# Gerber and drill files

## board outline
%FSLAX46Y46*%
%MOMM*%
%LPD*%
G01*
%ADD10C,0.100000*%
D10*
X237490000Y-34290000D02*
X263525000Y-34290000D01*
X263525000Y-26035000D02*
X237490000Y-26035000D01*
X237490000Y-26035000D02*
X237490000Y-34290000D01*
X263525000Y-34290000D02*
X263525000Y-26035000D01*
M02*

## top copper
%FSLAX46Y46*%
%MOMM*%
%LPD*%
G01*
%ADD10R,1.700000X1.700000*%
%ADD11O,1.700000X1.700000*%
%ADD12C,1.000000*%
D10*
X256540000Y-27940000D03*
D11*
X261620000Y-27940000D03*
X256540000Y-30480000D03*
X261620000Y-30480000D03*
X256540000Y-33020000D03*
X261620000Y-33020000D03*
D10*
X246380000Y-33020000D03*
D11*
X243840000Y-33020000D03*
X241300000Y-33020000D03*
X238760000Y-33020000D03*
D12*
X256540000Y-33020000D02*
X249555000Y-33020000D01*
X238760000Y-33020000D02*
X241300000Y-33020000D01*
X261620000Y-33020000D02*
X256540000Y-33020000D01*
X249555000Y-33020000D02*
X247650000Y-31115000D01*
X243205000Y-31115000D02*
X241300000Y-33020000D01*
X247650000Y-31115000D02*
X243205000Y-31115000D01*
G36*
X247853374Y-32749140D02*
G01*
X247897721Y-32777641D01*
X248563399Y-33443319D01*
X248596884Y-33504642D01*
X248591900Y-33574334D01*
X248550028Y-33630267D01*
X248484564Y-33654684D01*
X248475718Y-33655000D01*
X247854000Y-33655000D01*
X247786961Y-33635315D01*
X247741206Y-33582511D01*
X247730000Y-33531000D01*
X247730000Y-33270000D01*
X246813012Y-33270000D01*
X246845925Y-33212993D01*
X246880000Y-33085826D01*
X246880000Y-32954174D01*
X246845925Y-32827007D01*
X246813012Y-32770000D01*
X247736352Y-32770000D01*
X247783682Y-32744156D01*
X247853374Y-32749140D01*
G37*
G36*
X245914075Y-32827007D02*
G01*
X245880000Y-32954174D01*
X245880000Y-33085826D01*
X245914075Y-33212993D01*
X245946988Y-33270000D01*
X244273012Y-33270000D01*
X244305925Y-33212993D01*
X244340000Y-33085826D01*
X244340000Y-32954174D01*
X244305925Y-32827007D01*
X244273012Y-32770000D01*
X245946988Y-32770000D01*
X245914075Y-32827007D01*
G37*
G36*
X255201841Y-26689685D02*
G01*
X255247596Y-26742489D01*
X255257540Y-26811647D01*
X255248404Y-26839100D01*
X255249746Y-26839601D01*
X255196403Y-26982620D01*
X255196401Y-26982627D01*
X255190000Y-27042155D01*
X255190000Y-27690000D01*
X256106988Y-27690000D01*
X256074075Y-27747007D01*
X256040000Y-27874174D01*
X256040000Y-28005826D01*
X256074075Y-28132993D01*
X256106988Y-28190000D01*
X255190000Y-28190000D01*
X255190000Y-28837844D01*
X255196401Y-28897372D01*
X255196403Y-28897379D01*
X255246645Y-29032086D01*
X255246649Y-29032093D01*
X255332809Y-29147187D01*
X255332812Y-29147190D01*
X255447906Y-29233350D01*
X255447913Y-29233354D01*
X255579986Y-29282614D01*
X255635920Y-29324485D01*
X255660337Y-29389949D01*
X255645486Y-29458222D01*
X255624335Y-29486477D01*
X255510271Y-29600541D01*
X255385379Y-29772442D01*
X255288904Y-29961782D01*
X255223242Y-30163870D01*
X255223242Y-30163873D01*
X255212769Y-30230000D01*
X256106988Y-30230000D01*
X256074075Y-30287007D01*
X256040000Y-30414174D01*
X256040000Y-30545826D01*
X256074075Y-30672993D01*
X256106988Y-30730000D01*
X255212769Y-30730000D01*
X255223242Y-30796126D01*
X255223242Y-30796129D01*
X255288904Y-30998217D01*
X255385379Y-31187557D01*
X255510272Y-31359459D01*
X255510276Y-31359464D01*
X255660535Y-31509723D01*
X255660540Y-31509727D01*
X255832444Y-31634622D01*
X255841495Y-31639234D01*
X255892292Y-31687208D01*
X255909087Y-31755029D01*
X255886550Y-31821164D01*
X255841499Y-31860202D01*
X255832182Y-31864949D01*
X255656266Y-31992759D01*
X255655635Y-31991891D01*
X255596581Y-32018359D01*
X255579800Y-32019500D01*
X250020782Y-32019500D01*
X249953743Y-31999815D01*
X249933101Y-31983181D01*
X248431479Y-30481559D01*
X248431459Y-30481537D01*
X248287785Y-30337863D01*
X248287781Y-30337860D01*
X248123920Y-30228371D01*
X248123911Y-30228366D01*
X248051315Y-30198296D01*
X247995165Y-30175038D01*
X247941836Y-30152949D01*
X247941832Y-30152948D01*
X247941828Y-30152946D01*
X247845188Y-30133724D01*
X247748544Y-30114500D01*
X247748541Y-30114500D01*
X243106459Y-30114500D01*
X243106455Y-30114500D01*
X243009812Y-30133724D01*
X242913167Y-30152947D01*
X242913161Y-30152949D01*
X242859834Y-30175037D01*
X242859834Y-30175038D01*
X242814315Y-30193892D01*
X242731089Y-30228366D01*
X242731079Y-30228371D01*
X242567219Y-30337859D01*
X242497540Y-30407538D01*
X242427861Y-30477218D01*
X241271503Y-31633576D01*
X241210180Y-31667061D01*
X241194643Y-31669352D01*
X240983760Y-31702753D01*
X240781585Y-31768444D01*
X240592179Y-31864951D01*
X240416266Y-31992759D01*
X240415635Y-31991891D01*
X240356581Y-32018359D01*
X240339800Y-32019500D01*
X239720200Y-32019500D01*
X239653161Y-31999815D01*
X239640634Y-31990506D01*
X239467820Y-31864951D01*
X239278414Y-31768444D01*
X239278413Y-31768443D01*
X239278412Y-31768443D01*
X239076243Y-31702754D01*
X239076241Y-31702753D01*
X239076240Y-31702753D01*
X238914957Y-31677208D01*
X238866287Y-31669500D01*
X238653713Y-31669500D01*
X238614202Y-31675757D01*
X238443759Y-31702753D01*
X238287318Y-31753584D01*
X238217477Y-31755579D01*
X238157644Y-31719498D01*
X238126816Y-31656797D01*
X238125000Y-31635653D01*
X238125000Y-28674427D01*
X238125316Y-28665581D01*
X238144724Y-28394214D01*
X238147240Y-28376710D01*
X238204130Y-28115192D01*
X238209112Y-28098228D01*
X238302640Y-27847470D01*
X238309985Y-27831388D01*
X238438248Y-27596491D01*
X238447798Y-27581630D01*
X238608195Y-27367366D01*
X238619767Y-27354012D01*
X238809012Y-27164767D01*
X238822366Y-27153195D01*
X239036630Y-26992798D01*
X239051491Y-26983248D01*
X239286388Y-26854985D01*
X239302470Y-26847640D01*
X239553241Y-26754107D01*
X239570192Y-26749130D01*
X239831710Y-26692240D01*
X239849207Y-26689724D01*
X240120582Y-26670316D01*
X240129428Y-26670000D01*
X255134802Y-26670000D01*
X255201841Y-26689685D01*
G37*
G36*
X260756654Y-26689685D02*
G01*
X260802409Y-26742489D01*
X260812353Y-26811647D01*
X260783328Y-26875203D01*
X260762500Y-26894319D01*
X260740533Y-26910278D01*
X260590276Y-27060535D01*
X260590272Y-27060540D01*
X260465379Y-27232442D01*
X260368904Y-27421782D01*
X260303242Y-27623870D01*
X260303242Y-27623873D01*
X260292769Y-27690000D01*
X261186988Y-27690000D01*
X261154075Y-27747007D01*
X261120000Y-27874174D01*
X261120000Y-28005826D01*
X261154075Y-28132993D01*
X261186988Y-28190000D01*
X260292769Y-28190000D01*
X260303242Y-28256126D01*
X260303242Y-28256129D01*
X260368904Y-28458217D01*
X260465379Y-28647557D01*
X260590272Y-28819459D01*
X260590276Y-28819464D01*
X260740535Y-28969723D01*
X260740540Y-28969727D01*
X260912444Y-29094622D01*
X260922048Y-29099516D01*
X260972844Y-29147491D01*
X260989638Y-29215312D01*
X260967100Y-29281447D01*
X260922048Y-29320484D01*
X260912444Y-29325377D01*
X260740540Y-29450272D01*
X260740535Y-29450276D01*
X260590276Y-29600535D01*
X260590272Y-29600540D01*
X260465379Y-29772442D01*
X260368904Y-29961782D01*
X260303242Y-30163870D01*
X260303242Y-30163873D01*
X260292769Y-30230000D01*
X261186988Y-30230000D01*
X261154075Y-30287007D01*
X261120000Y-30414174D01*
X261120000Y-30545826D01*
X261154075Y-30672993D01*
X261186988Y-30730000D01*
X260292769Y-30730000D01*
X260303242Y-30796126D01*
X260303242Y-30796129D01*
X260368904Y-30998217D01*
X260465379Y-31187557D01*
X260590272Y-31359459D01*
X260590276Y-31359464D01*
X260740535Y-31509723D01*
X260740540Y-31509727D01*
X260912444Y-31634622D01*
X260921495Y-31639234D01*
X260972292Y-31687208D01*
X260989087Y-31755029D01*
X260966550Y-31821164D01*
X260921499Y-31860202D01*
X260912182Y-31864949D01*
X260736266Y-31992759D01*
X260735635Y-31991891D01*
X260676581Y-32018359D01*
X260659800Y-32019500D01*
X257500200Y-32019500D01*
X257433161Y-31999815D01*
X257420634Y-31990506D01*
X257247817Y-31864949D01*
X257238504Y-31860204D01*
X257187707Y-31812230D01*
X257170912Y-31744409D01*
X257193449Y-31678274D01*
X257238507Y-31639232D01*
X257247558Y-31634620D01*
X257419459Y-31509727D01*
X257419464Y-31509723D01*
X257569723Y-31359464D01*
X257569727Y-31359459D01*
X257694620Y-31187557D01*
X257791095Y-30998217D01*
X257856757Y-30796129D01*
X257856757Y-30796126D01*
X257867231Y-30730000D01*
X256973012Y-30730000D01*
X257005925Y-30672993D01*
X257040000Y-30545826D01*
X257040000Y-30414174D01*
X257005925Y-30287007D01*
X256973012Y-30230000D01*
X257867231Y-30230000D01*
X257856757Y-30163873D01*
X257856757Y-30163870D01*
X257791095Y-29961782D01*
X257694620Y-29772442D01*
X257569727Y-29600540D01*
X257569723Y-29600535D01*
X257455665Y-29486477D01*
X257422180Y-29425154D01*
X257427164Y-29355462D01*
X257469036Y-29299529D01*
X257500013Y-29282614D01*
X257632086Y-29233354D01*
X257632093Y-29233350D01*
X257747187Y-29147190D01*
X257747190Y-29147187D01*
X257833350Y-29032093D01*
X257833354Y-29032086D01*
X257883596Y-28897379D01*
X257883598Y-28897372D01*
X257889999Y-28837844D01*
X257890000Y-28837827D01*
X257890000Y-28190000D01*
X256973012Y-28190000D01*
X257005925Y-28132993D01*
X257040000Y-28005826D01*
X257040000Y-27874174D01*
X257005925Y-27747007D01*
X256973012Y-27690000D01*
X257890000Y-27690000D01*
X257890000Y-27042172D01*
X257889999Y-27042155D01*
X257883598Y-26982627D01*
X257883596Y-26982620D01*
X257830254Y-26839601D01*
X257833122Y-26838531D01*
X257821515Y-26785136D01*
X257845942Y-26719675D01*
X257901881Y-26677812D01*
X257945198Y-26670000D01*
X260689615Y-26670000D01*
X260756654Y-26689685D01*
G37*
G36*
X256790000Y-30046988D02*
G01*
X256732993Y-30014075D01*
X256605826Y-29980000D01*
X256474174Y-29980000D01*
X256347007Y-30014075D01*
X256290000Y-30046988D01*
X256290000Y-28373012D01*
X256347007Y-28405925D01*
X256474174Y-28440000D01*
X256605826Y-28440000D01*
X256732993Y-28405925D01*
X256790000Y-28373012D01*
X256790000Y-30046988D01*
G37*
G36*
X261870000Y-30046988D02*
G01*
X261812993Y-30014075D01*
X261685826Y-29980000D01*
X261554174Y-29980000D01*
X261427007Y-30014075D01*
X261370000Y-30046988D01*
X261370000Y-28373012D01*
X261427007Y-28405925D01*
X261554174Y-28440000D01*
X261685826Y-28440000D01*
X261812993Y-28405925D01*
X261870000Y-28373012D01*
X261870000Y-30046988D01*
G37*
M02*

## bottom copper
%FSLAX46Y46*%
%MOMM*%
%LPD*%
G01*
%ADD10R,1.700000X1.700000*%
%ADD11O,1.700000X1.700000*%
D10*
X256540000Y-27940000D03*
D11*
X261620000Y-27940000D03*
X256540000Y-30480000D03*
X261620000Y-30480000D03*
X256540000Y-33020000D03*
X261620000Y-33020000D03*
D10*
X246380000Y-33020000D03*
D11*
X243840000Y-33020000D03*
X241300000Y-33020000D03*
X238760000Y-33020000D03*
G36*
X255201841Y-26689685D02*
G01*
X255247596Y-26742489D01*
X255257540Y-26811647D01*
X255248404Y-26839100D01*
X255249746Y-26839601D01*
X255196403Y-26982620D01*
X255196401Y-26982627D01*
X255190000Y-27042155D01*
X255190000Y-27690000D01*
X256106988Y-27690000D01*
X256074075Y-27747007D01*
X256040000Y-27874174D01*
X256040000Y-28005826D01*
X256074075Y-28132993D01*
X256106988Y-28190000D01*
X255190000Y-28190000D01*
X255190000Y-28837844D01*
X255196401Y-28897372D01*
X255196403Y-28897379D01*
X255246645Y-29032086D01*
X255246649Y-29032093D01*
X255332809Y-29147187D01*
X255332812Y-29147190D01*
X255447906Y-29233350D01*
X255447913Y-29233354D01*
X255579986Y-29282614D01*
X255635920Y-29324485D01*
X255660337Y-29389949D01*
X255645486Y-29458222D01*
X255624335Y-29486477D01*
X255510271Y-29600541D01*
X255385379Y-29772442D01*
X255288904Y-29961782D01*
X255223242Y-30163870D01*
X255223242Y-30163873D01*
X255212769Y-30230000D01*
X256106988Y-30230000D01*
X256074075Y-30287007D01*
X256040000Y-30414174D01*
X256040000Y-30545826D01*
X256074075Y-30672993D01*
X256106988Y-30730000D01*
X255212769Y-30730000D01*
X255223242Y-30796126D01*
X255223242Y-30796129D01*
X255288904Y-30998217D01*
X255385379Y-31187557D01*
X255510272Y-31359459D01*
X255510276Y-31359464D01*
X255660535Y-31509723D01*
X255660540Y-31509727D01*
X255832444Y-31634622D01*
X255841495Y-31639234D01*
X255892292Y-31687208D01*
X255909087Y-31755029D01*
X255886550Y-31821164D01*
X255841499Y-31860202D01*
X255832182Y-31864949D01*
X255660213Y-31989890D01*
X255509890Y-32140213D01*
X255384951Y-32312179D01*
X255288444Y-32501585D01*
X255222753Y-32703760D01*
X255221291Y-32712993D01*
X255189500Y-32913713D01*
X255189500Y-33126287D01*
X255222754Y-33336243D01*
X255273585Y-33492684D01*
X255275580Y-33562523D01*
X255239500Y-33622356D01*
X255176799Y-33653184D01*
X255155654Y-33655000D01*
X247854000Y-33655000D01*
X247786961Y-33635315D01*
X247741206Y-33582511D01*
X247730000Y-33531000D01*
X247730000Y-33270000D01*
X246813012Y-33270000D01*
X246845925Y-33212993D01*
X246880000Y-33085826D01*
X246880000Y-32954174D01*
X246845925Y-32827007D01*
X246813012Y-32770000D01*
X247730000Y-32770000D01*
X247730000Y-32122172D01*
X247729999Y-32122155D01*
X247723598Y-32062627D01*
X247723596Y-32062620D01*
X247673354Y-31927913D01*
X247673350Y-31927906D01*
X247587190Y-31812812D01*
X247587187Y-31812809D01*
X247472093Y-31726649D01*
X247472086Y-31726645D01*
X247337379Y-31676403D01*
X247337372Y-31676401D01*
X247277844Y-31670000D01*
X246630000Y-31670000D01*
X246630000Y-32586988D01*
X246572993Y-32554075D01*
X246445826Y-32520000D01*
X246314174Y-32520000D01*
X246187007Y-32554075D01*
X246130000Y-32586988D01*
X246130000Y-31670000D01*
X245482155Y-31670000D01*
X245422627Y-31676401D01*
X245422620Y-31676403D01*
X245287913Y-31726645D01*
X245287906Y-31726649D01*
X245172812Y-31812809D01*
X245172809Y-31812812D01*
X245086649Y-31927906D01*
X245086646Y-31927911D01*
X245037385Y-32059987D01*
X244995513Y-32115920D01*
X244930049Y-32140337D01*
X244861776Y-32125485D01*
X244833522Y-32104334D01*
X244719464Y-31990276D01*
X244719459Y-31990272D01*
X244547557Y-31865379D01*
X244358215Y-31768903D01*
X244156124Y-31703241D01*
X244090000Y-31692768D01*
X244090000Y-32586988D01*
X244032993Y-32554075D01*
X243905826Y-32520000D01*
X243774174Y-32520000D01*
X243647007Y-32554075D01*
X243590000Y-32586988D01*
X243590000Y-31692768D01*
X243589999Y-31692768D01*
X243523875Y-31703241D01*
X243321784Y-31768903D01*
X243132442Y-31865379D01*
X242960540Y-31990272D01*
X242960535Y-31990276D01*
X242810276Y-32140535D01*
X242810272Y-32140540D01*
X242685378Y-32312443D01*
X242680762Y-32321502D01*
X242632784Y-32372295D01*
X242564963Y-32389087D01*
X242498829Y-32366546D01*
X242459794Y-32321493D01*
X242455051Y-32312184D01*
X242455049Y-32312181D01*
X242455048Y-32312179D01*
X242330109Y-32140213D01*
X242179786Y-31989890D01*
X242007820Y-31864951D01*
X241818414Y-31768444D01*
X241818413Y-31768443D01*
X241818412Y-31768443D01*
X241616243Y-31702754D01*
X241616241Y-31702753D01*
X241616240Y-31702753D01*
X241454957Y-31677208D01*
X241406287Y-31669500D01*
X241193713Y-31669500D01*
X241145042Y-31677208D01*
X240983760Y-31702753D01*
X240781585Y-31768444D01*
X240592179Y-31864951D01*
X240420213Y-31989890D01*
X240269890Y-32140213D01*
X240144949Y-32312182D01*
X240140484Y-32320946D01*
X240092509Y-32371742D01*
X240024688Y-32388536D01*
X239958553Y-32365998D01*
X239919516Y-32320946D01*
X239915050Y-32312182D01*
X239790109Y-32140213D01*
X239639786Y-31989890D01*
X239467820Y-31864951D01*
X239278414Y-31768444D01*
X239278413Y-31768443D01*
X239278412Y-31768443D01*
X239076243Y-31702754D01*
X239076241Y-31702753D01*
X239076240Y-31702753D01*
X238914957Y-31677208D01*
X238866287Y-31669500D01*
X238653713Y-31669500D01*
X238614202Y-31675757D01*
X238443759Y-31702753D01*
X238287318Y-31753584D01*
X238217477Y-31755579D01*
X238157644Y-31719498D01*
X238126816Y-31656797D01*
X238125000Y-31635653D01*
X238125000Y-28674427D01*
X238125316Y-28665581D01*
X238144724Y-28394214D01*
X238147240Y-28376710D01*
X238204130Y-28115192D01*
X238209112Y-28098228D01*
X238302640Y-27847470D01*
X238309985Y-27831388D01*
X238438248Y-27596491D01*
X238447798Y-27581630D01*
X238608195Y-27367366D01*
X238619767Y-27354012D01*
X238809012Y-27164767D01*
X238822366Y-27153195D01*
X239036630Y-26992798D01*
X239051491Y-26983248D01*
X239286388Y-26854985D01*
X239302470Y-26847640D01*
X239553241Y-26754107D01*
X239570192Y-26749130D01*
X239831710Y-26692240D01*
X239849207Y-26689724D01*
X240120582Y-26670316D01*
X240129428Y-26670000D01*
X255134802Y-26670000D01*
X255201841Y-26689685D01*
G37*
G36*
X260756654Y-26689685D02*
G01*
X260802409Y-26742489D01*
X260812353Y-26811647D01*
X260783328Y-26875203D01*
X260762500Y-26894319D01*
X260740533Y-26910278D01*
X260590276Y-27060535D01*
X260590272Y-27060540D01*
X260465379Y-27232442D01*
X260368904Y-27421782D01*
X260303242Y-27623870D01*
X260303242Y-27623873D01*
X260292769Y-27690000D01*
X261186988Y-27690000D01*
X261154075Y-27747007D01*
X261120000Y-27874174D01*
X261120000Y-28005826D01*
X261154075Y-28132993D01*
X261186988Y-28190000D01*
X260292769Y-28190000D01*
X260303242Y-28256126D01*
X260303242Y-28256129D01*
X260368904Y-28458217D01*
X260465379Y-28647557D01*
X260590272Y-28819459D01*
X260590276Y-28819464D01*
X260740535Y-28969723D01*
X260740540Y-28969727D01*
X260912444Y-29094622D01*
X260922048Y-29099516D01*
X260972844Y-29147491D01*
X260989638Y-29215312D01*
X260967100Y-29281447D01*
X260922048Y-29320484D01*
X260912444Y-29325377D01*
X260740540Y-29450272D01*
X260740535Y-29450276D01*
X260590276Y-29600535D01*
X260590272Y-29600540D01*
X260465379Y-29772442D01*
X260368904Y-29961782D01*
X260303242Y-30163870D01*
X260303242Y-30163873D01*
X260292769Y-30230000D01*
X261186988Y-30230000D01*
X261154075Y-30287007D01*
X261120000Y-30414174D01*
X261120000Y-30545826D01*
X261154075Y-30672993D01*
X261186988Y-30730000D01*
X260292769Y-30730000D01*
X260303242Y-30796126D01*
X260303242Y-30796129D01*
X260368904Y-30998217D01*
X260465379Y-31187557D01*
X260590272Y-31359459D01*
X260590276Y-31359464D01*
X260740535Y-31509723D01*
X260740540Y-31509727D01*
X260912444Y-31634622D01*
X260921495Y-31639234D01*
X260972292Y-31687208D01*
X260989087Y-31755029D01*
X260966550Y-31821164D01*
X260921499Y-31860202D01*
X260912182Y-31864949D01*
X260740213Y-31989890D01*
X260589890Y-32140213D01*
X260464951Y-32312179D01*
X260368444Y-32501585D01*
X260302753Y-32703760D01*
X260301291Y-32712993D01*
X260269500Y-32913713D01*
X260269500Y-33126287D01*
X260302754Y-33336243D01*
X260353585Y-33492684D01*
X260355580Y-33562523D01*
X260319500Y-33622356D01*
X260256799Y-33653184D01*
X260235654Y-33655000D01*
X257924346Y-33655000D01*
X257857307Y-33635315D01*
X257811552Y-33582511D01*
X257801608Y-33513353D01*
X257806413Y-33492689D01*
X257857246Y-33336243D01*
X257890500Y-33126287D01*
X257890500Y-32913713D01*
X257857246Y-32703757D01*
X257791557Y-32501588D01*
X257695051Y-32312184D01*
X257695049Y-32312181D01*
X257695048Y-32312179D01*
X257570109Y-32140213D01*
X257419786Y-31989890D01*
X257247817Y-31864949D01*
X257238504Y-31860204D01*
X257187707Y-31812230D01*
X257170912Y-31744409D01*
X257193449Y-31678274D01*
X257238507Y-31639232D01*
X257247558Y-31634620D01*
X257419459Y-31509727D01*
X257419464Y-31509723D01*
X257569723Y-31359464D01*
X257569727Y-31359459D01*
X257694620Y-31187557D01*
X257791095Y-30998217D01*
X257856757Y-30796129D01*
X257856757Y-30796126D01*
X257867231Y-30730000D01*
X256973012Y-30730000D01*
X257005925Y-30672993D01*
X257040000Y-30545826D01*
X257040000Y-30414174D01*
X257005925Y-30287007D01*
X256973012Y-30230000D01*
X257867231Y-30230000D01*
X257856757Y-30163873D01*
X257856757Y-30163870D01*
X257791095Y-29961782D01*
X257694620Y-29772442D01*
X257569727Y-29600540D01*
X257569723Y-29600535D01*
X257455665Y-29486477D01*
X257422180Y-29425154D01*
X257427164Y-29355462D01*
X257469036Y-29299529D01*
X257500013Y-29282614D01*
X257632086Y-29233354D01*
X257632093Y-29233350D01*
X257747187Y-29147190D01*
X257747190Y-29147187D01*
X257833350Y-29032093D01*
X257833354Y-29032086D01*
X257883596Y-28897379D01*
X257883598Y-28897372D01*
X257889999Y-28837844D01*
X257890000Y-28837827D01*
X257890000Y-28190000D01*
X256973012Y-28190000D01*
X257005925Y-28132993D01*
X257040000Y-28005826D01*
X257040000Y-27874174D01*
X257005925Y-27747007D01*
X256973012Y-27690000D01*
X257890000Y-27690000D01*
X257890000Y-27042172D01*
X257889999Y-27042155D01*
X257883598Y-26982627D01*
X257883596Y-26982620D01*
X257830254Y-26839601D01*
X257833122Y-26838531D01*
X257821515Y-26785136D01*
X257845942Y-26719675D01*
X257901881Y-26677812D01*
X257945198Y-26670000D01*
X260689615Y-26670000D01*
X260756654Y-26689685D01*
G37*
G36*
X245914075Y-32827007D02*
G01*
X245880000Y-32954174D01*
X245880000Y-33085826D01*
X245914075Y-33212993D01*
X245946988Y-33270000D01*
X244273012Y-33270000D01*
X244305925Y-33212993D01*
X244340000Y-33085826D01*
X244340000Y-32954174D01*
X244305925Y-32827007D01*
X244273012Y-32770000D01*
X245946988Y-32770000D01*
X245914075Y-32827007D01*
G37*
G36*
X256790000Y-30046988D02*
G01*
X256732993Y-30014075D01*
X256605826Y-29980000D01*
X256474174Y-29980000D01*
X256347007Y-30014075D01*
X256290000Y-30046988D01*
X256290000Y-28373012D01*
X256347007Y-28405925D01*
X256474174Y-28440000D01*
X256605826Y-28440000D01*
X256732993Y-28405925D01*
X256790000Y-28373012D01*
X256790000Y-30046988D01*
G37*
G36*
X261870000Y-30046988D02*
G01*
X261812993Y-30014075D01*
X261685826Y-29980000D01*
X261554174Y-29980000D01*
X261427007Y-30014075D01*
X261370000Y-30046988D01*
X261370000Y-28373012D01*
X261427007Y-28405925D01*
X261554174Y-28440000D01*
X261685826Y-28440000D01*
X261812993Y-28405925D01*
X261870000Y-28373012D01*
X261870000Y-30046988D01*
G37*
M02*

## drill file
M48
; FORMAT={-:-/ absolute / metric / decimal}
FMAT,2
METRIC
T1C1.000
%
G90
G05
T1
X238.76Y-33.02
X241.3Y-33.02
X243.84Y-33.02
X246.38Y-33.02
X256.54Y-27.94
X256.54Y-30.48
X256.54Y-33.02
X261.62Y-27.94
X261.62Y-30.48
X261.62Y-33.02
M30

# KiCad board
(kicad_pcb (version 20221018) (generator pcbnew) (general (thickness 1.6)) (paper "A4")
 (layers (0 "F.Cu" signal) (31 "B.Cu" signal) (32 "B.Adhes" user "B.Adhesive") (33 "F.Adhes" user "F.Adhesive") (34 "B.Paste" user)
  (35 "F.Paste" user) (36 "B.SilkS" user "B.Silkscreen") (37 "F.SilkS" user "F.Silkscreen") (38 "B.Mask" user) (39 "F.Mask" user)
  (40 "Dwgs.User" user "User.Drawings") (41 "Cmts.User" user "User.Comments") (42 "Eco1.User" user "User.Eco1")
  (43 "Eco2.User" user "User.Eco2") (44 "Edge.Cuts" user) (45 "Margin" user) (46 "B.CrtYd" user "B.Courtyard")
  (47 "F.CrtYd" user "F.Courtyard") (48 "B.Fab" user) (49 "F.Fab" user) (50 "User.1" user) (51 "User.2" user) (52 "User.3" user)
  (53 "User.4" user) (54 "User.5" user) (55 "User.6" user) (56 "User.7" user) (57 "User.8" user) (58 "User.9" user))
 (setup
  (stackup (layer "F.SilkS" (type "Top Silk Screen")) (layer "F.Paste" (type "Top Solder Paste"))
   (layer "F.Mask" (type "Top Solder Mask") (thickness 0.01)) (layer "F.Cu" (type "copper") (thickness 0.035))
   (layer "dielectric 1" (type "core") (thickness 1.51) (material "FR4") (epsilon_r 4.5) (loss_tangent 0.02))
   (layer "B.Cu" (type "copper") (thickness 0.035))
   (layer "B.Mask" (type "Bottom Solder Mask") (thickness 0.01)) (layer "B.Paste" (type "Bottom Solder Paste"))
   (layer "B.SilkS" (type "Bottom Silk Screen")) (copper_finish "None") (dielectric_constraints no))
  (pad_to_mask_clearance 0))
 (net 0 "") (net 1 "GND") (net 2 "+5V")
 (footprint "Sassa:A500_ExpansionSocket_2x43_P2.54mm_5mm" (layer "F.Cu") (at 256.54 27.94)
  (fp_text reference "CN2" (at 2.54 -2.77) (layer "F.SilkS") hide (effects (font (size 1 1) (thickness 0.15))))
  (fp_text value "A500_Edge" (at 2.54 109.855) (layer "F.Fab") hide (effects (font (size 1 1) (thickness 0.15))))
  (pad "1" thru_hole rect (at 0 0) (size 1.7 1.7) (drill 1) (layers "*.Cu" "*.Mask") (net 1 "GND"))
  (pad "2" thru_hole oval (at 5.08 0) (size 1.7 1.7) (drill 1) (layers "*.Cu" "*.Mask") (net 1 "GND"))
  (pad "3" thru_hole oval (at 0 2.54) (size 1.7 1.7) (drill 1) (layers "*.Cu" "*.Mask") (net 1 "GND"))
  (pad "4" thru_hole oval (at 5.08 2.54) (size 1.7 1.7) (drill 1) (layers "*.Cu" "*.Mask") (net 1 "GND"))
  (pad "5" thru_hole oval (at 0 5.08) (size 1.7 1.7) (drill 1) (layers "*.Cu" "*.Mask") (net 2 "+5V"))
  (pad "6" thru_hole oval (at 5.08 5.08) (size 1.7 1.7) (drill 1) (layers "*.Cu" "*.Mask") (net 2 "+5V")))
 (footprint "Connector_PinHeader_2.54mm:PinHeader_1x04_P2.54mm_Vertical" (layer "F.Cu") (at 246.38 33.02 -90)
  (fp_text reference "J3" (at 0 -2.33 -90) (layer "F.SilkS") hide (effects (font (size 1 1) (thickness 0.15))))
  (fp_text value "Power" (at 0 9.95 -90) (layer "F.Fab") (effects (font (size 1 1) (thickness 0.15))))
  (pad "1" thru_hole rect (at 0 0 270) (size 1.7 1.7) (drill 1) (layers "*.Cu" "*.Mask") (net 1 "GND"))
  (pad "2" thru_hole oval (at 0 2.54 270) (size 1.7 1.7) (drill 1) (layers "*.Cu" "*.Mask") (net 1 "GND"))
  (pad "3" thru_hole oval (at 0 5.08 270) (size 1.7 1.7) (drill 1) (layers "*.Cu" "*.Mask") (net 2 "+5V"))
  (pad "4" thru_hole oval (at 0 7.62 270) (size 1.7 1.7) (drill 1) (layers "*.Cu" "*.Mask") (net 2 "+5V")))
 (gr_line (start 237.49 34.29) (end 263.525 34.29) (stroke (width 0.1) (type default)) (layer "Edge.Cuts"))
 (gr_line (start 263.525 26.035) (end 237.49 26.035) (stroke (width 0.1) (type default)) (layer "Edge.Cuts"))
 (gr_line (start 237.49 26.035) (end 237.49 34.29) (stroke (width 0.1) (type default)) (layer "Edge.Cuts"))
 (gr_line (start 263.525 34.29) (end 263.525 26.035) (stroke (width 0.1) (type default)) (layer "Edge.Cuts"))
 (segment (start 256.54 33.02) (end 249.555 33.02) (width 1) (layer "F.Cu") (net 2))
 (segment (start 238.76 33.02) (end 241.3 33.02) (width 1) (layer "F.Cu") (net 2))
 (segment (start 261.62 33.02) (end 256.54 33.02) (width 1) (layer "F.Cu") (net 2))
 (segment (start 249.555 33.02) (end 247.65 31.115) (width 1) (layer "F.Cu") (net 2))
 (segment (start 243.205 31.115) (end 241.3 33.02) (width 1) (layer "F.Cu") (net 2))
 (segment (start 247.65 31.115) (end 243.205 31.115) (width 1) (layer "F.Cu") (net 2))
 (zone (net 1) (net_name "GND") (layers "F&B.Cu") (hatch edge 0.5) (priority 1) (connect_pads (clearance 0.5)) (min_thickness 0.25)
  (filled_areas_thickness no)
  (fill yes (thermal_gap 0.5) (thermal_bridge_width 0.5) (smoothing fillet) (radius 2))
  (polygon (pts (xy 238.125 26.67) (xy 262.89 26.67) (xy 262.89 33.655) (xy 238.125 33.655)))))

